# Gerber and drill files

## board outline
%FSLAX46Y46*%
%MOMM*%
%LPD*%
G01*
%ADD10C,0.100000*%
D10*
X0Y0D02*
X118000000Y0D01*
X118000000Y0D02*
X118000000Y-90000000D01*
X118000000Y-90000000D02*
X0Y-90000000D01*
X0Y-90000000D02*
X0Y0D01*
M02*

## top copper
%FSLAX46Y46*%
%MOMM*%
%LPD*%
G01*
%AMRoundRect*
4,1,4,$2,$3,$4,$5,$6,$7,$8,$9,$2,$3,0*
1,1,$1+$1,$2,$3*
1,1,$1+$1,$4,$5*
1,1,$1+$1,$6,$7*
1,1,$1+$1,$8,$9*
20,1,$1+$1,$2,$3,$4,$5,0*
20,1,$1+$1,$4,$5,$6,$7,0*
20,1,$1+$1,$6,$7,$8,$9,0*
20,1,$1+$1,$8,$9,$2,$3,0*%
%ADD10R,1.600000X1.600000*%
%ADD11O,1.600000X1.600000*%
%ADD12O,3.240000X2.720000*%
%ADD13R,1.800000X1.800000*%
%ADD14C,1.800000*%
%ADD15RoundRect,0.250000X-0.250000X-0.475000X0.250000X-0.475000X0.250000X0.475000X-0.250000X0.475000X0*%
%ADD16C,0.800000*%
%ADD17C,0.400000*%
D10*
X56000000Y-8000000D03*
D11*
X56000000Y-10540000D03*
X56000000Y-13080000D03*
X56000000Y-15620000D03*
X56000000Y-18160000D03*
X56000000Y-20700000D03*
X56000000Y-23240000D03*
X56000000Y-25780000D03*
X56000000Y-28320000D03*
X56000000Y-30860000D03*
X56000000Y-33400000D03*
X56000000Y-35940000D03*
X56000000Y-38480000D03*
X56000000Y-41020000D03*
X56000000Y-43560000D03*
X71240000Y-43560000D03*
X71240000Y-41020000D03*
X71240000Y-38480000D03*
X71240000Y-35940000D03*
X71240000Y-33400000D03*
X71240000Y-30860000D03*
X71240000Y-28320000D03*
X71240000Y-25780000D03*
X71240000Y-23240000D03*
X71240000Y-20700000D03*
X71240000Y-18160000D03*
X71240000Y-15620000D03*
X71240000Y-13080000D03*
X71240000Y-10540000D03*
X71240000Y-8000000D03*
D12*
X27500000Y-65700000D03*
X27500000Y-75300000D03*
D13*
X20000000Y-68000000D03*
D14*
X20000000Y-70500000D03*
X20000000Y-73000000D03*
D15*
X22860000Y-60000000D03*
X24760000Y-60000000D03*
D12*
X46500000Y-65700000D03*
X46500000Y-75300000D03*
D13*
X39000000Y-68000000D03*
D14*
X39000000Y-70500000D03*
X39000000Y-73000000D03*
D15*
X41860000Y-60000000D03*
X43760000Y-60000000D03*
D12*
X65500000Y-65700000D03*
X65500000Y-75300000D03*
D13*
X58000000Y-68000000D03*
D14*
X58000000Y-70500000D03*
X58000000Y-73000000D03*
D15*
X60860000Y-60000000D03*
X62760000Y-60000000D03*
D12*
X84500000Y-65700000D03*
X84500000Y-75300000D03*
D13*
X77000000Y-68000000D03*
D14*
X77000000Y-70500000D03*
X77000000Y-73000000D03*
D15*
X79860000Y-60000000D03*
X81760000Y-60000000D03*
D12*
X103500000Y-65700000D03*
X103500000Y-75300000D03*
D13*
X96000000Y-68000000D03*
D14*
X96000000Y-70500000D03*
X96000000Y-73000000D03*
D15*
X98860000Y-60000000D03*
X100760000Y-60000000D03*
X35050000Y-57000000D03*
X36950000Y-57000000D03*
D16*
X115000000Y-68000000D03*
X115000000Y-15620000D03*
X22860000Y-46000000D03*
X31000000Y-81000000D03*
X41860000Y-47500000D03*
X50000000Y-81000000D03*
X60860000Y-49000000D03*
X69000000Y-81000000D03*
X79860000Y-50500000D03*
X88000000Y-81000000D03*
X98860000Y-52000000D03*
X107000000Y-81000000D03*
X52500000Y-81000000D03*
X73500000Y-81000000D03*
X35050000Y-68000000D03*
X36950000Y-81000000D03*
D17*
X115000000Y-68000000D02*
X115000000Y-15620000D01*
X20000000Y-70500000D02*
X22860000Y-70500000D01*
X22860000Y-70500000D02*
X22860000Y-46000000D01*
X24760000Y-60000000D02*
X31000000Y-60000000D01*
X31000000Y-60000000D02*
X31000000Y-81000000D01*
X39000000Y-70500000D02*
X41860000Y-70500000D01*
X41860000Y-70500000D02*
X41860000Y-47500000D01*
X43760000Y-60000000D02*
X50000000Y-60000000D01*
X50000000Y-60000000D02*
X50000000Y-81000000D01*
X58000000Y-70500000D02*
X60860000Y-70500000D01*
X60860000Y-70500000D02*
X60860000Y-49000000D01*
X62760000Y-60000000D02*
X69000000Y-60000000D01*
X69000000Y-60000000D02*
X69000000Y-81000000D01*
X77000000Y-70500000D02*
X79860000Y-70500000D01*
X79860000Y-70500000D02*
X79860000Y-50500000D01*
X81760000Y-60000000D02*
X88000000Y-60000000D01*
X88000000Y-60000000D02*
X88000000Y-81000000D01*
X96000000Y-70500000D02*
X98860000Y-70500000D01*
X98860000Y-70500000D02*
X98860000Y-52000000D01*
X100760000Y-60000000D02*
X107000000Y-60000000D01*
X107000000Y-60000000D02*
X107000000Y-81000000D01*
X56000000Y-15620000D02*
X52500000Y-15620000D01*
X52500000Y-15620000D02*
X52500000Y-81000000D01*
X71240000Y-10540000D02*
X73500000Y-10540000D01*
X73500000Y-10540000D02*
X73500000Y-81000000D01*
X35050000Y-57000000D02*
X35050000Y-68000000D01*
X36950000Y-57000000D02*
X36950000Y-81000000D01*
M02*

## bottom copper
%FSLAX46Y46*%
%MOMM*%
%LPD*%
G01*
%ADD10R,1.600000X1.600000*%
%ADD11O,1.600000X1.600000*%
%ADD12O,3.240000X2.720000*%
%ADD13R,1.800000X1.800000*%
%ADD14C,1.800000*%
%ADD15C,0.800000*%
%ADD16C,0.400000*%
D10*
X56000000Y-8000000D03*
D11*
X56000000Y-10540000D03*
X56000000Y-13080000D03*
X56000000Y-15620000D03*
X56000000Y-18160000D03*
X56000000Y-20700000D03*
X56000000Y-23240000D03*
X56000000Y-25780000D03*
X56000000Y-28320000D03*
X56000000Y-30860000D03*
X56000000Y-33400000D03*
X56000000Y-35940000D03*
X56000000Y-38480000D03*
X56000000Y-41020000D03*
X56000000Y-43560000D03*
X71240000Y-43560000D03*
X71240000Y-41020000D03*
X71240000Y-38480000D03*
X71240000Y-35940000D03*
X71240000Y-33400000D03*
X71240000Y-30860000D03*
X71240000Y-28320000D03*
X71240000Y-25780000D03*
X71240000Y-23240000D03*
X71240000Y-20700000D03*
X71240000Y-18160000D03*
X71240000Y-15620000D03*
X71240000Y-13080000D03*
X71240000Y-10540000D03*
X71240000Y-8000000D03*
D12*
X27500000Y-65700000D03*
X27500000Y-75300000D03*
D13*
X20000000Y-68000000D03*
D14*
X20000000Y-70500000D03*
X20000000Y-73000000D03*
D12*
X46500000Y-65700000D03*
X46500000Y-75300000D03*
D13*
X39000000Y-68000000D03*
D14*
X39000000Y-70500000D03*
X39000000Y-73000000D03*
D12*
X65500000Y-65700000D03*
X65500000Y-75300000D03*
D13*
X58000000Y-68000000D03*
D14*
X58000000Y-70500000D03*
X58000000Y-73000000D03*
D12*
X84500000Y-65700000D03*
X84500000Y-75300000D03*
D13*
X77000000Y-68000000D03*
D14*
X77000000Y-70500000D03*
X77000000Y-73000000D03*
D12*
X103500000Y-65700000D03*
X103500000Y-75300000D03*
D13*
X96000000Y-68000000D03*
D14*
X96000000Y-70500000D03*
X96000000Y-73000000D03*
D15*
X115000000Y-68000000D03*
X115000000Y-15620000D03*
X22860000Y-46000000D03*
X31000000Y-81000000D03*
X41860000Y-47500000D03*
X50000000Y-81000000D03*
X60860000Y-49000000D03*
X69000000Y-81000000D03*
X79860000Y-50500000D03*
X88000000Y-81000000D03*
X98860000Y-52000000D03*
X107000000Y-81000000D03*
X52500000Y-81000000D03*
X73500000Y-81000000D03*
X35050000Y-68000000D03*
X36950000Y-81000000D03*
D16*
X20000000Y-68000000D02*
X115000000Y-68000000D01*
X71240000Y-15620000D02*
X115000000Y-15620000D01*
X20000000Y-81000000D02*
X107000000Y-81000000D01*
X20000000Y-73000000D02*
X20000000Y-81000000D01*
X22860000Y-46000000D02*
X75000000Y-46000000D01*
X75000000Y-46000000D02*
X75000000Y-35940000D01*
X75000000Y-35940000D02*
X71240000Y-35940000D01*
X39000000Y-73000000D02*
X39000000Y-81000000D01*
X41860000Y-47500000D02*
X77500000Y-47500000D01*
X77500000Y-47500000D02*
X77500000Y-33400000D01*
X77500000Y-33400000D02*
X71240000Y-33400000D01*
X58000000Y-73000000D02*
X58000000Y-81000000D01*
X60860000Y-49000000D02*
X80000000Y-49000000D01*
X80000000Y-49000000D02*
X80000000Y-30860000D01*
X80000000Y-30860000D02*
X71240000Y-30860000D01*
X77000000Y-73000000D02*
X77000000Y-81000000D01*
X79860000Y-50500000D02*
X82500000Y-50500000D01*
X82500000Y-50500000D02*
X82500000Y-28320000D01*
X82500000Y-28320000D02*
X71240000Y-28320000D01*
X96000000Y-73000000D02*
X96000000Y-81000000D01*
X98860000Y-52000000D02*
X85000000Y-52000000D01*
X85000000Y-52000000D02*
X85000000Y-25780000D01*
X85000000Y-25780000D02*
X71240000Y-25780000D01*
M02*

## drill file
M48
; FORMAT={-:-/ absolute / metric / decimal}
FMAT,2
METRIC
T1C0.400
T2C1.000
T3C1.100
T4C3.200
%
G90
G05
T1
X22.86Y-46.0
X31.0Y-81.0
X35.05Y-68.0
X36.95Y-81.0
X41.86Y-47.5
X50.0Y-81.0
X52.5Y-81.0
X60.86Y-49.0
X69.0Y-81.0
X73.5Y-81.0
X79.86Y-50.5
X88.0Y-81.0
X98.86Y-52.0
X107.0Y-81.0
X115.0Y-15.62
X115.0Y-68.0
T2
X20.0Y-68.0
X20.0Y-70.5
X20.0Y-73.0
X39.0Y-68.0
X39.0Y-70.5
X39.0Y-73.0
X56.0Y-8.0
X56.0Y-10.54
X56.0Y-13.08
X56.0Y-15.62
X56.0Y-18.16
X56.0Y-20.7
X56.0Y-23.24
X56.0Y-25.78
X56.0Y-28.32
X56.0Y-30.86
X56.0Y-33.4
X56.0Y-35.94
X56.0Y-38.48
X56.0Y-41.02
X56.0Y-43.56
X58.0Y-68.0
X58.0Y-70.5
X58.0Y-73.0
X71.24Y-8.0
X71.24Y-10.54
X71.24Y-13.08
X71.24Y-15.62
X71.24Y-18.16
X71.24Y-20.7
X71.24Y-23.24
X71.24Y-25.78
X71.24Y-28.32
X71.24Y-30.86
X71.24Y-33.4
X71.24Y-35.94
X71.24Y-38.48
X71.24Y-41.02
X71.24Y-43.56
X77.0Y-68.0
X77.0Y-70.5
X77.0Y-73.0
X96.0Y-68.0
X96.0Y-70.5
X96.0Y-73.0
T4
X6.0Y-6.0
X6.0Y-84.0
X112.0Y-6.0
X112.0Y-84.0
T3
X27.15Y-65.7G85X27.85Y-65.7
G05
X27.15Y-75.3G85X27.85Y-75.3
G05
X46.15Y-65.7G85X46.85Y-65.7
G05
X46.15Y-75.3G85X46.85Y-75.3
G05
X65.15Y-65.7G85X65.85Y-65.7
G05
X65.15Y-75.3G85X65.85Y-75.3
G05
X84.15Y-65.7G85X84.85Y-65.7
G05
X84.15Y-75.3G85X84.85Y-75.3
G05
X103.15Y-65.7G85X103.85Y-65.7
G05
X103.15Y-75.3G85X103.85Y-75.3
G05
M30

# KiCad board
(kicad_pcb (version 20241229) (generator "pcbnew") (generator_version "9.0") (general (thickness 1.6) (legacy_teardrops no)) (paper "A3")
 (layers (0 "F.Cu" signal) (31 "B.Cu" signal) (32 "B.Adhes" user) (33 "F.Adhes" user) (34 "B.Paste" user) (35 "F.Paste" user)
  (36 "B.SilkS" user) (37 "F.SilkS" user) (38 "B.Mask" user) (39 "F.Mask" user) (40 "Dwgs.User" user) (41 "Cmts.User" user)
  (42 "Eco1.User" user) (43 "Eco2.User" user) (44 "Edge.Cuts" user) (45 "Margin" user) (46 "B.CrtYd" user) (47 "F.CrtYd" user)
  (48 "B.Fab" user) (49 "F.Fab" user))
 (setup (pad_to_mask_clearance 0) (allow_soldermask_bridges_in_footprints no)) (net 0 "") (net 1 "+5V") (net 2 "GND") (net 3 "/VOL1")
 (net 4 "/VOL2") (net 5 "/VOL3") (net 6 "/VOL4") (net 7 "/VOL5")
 (gr_line (start 0 0) (end 118 0) (stroke (width 0.1) (type solid)) (layer "Edge.Cuts"))
 (gr_line (start 118 0) (end 118 90) (stroke (width 0.1) (type solid)) (layer "Edge.Cuts"))
 (gr_line (start 118 90) (end 0 90) (stroke (width 0.1) (type solid)) (layer "Edge.Cuts"))
 (gr_line (start 0 90) (end 0 0) (stroke (width 0.1) (type solid)) (layer "Edge.Cuts"))
 (segment (start 20 68) (end 115 68) (width 0.4) (layer "B.Cu") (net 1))
 (segment (start 71.24 15.62) (end 115 15.62) (width 0.4) (layer "B.Cu") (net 1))
 (segment (start 20 81) (end 107 81) (width 0.4) (layer "B.Cu") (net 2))
 (segment (start 20 73) (end 20 81) (width 0.4) (layer "B.Cu") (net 2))
 (segment (start 22.86 46) (end 75 46) (width 0.4) (layer "B.Cu") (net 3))
 (segment (start 75 46) (end 75 35.94) (width 0.4) (layer "B.Cu") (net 3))
 (segment (start 75 35.94) (end 71.24 35.94) (width 0.4) (layer "B.Cu") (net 3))
 (segment (start 39 73) (end 39 81) (width 0.4) (layer "B.Cu") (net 2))
 (segment (start 41.86 47.5) (end 77.5 47.5) (width 0.4) (layer "B.Cu") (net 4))
 (segment (start 77.5 47.5) (end 77.5 33.4) (width 0.4) (layer "B.Cu") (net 4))
 (segment (start 77.5 33.4) (end 71.24 33.4) (width 0.4) (layer "B.Cu") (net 4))
 (segment (start 58 73) (end 58 81) (width 0.4) (layer "B.Cu") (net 2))
 (segment (start 60.86 49) (end 80 49) (width 0.4) (layer "B.Cu") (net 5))
 (segment (start 80 49) (end 80 30.86) (width 0.4) (layer "B.Cu") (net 5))
 (segment (start 80 30.86) (end 71.24 30.86) (width 0.4) (layer "B.Cu") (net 5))
 (segment (start 77 73) (end 77 81) (width 0.4) (layer "B.Cu") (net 2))
 (segment (start 79.86 50.5) (end 82.5 50.5) (width 0.4) (layer "B.Cu") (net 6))
 (segment (start 82.5 50.5) (end 82.5 28.32) (width 0.4) (layer "B.Cu") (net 6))
 (segment (start 82.5 28.32) (end 71.24 28.32) (width 0.4) (layer "B.Cu") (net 6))
 (segment (start 96 73) (end 96 81) (width 0.4) (layer "B.Cu") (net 2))
 (segment (start 98.86 52) (end 85 52) (width 0.4) (layer "B.Cu") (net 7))
 (segment (start 85 52) (end 85 25.78) (width 0.4) (layer "B.Cu") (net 7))
 (segment (start 85 25.78) (end 71.24 25.78) (width 0.4) (layer "B.Cu") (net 7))
 (segment (start 115 68) (end 115 15.62) (width 0.4) (layer "F.Cu") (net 1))
 (segment (start 20 70.5) (end 22.86 70.5) (width 0.4) (layer "F.Cu") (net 3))
 (segment (start 22.86 70.5) (end 22.86 46) (width 0.4) (layer "F.Cu") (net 3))
 (segment (start 24.76 60) (end 31 60) (width 0.4) (layer "F.Cu") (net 2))
 (segment (start 31 60) (end 31 81) (width 0.4) (layer "F.Cu") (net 2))
 (segment (start 39 70.5) (end 41.86 70.5) (width 0.4) (layer "F.Cu") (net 4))
 (segment (start 41.86 70.5) (end 41.86 47.5) (width 0.4) (layer "F.Cu") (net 4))
 (segment (start 43.76 60) (end 50 60) (width 0.4) (layer "F.Cu") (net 2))
 (segment (start 50 60) (end 50 81) (width 0.4) (layer "F.Cu") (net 2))
 (segment (start 58 70.5) (end 60.86 70.5) (width 0.4) (layer "F.Cu") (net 5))
 (segment (start 60.86 70.5) (end 60.86 49) (width 0.4) (layer "F.Cu") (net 5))
 (segment (start 62.76 60) (end 69 60) (width 0.4) (layer "F.Cu") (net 2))
 (segment (start 69 60) (end 69 81) (width 0.4) (layer "F.Cu") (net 2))
 (segment (start 77 70.5) (end 79.86 70.5) (width 0.4) (layer "F.Cu") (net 6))
 (segment (start 79.86 70.5) (end 79.86 50.5) (width 0.4) (layer "F.Cu") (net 6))
 (segment (start 81.76 60) (end 88 60) (width 0.4) (layer "F.Cu") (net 2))
 (segment (start 88 60) (end 88 81) (width 0.4) (layer "F.Cu") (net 2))
 (segment (start 96 70.5) (end 98.86 70.5) (width 0.4) (layer "F.Cu") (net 7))
 (segment (start 98.86 70.5) (end 98.86 52) (width 0.4) (layer "F.Cu") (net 7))
 (segment (start 100.76 60) (end 107 60) (width 0.4) (layer "F.Cu") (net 2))
 (segment (start 107 60) (end 107 81) (width 0.4) (layer "F.Cu") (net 2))
 (segment (start 56 15.62) (end 52.5 15.62) (width 0.4) (layer "F.Cu") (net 2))
 (segment (start 52.5 15.62) (end 52.5 81) (width 0.4) (layer "F.Cu") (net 2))
 (segment (start 71.24 10.54) (end 73.5 10.54) (width 0.4) (layer "F.Cu") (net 2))
 (segment (start 73.5 10.54) (end 73.5 81) (width 0.4) (layer "F.Cu") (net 2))
 (segment (start 35.05 57) (end 35.05 68) (width 0.4) (layer "F.Cu") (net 1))
 (segment (start 36.95 57) (end 36.95 81) (width 0.4) (layer "F.Cu") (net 2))
 (via (at 115 68) (size 0.8) (drill 0.4) (layers "F.Cu" "B.Cu") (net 1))
 (via (at 115 15.62) (size 0.8) (drill 0.4) (layers "F.Cu" "B.Cu") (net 1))
 (via (at 22.86 46) (size 0.8) (drill 0.4) (layers "F.Cu" "B.Cu") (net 3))
 (via (at 31 81) (size 0.8) (drill 0.4) (layers "F.Cu" "B.Cu") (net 2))
 (via (at 41.86 47.5) (size 0.8) (drill 0.4) (layers "F.Cu" "B.Cu") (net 4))
 (via (at 50 81) (size 0.8) (drill 0.4) (layers "F.Cu" "B.Cu") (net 2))
 (via (at 60.86 49) (size 0.8) (drill 0.4) (layers "F.Cu" "B.Cu") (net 5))
 (via (at 69 81) (size 0.8) (drill 0.4) (layers "F.Cu" "B.Cu") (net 2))
 (via (at 79.86 50.5) (size 0.8) (drill 0.4) (layers "F.Cu" "B.Cu") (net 6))
 (via (at 88 81) (size 0.8) (drill 0.4) (layers "F.Cu" "B.Cu") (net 2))
 (via (at 98.86 52) (size 0.8) (drill 0.4) (layers "F.Cu" "B.Cu") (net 7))
 (via (at 107 81) (size 0.8) (drill 0.4) (layers "F.Cu" "B.Cu") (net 2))
 (via (at 52.5 81) (size 0.8) (drill 0.4) (layers "F.Cu" "B.Cu") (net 2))
 (via (at 73.5 81) (size 0.8) (drill 0.4) (layers "F.Cu" "B.Cu") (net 2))
 (via (at 35.05 68) (size 0.8) (drill 0.4) (layers "F.Cu" "B.Cu") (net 1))
 (via (at 36.95 81) (size 0.8) (drill 0.4) (layers "F.Cu" "B.Cu") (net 2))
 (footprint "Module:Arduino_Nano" (at 56 8 0) (layer "F.Cu")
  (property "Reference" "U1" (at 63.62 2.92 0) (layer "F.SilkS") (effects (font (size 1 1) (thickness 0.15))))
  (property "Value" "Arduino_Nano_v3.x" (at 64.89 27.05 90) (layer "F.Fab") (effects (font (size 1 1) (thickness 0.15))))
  (pad "1" thru_hole rect (at 0 0) (size 1.6 1.6) (drill 1) (layers "*.Cu" "*.Mask") (remove_unused_layers no))
  (pad "2" thru_hole oval (at 0 2.54) (size 1.6 1.6) (drill 1) (layers "*.Cu" "*.Mask") (remove_unused_layers no))
  (pad "3" thru_hole oval (at 0 5.08) (size 1.6 1.6) (drill 1) (layers "*.Cu" "*.Mask") (remove_unused_layers no))
  (pad "4" thru_hole oval (at 0 7.62) (size 1.6 1.6) (drill 1) (layers "*.Cu" "*.Mask") (remove_unused_layers no) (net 2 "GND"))
  (pad "5" thru_hole oval (at 0 10.16) (size 1.6 1.6) (drill 1) (layers "*.Cu" "*.Mask") (remove_unused_layers no))
  (pad "6" thru_hole oval (at 0 12.7) (size 1.6 1.6) (drill 1) (layers "*.Cu" "*.Mask") (remove_unused_layers no))
  (pad "7" thru_hole oval (at 0 15.24) (size 1.6 1.6) (drill 1) (layers "*.Cu" "*.Mask") (remove_unused_layers no))
  (pad "8" thru_hole oval (at 0 17.78) (size 1.6 1.6) (drill 1) (layers "*.Cu" "*.Mask") (remove_unused_layers no))
  (pad "9" thru_hole oval (at 0 20.32) (size 1.6 1.6) (drill 1) (layers "*.Cu" "*.Mask") (remove_unused_layers no))
  (pad "10" thru_hole oval (at 0 22.86) (size 1.6 1.6) (drill 1) (layers "*.Cu" "*.Mask") (remove_unused_layers no))
  (pad "11" thru_hole oval (at 0 25.4) (size 1.6 1.6) (drill 1) (layers "*.Cu" "*.Mask") (remove_unused_layers no))
  (pad "12" thru_hole oval (at 0 27.94) (size 1.6 1.6) (drill 1) (layers "*.Cu" "*.Mask") (remove_unused_layers no))
  (pad "13" thru_hole oval (at 0 30.48) (size 1.6 1.6) (drill 1) (layers "*.Cu" "*.Mask") (remove_unused_layers no))
  (pad "14" thru_hole oval (at 0 33.02) (size 1.6 1.6) (drill 1) (layers "*.Cu" "*.Mask") (remove_unused_layers no))
  (pad "15" thru_hole oval (at 0 35.56) (size 1.6 1.6) (drill 1) (layers "*.Cu" "*.Mask") (remove_unused_layers no))
  (pad "16" thru_hole oval (at 15.24 35.56) (size 1.6 1.6) (drill 1) (layers "*.Cu" "*.Mask") (remove_unused_layers no))
  (pad "17" thru_hole oval (at 15.24 33.02) (size 1.6 1.6) (drill 1) (layers "*.Cu" "*.Mask") (remove_unused_layers no))
  (pad "18" thru_hole oval (at 15.24 30.48) (size 1.6 1.6) (drill 1) (layers "*.Cu" "*.Mask") (remove_unused_layers no))
  (pad "19" thru_hole oval (at 15.24 27.94) (size 1.6 1.6) (drill 1) (layers "*.Cu" "*.Mask") (remove_unused_layers no) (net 3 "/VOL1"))
  (pad "20" thru_hole oval (at 15.24 25.4) (size 1.6 1.6) (drill 1) (layers "*.Cu" "*.Mask") (remove_unused_layers no) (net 4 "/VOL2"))
  (pad "21" thru_hole oval (at 15.24 22.86) (size 1.6 1.6) (drill 1) (layers "*.Cu" "*.Mask") (remove_unused_layers no) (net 5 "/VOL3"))
  (pad "22" thru_hole oval (at 15.24 20.32) (size 1.6 1.6) (drill 1) (layers "*.Cu" "*.Mask") (remove_unused_layers no) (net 6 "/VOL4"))
  (pad "23" thru_hole oval (at 15.24 17.78) (size 1.6 1.6) (drill 1) (layers "*.Cu" "*.Mask") (remove_unused_layers no) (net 7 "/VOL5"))
  (pad "24" thru_hole oval (at 15.24 15.24) (size 1.6 1.6) (drill 1) (layers "*.Cu" "*.Mask") (remove_unused_layers no))
  (pad "25" thru_hole oval (at 15.24 12.7) (size 1.6 1.6) (drill 1) (layers "*.Cu" "*.Mask") (remove_unused_layers no))
  (pad "26" thru_hole oval (at 15.24 10.16) (size 1.6 1.6) (drill 1) (layers "*.Cu" "*.Mask") (remove_unused_layers no))
  (pad "27" thru_hole oval (at 15.24 7.62) (size 1.6 1.6) (drill 1) (layers "*.Cu" "*.Mask") (remove_unused_layers no) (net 1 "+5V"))
  (pad "28" thru_hole oval (at 15.24 5.08) (size 1.6 1.6) (drill 1) (layers "*.Cu" "*.Mask") (remove_unused_layers no))
  (pad "29" thru_hole oval (at 15.24 2.54) (size 1.6 1.6) (drill 1) (layers "*.Cu" "*.Mask") (remove_unused_layers no) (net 2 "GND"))
  (pad "30" thru_hole oval (at 15.24 0) (size 1.6 1.6) (drill 1) (layers "*.Cu" "*.Mask") (remove_unused_layers no)))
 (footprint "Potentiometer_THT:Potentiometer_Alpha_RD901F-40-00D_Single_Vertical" (at 20 68 0) (layer "F.Cu")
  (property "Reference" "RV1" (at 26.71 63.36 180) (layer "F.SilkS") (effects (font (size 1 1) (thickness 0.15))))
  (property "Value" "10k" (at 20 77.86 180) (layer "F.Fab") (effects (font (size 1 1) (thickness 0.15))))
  (pad "" thru_hole oval (at 7.5 -2.3 90) (size 2.72 3.24) (drill oval 1.1 1.8) (layers "*.Cu" "*.Mask") (remove_unused_layers no))
  (pad "" thru_hole oval (at 7.5 7.3 90) (size 2.72 3.24) (drill oval 1.1 1.8) (layers "*.Cu" "*.Mask") (remove_unused_layers no))
  (pad "1" thru_hole rect (at 0 0 90) (size 1.8 1.8) (drill 1) (layers "*.Cu" "*.Mask") (remove_unused_layers no) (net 1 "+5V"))
  (pad "2" thru_hole circle (at 0 2.5 90) (size 1.8 1.8) (drill 1) (layers "*.Cu" "*.Mask") (remove_unused_layers no) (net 3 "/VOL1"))
  (pad "3" thru_hole circle (at 0 5 90) (size 1.8 1.8) (drill 1) (layers "*.Cu" "*.Mask") (remove_unused_layers no) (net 2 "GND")))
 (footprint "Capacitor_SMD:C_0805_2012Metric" (at 23.81 60 0) (layer "F.Cu")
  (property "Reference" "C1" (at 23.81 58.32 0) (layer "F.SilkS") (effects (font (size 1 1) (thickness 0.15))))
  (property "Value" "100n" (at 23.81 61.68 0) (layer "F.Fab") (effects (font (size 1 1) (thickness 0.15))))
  (pad "1" smd roundrect (at -0.95 0) (size 1 1.45) (layers "F.Cu" "F.Mask" "F.Paste") (roundrect_rratio 0.25) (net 3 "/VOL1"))
  (pad "2" smd roundrect (at 0.95 0) (size 1 1.45) (layers "F.Cu" "F.Mask" "F.Paste") (roundrect_rratio 0.25) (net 2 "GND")))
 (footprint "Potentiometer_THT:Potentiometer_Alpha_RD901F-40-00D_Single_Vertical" (at 39 68 0) (layer "F.Cu")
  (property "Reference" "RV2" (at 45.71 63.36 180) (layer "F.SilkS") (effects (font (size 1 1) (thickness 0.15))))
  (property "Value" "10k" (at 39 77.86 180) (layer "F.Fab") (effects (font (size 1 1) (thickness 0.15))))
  (pad "" thru_hole oval (at 7.5 -2.3 90) (size 2.72 3.24) (drill oval 1.1 1.8) (layers "*.Cu" "*.Mask") (remove_unused_layers no))
  (pad "" thru_hole oval (at 7.5 7.3 90) (size 2.72 3.24) (drill oval 1.1 1.8) (layers "*.Cu" "*.Mask") (remove_unused_layers no))
  (pad "1" thru_hole rect (at 0 0 90) (size 1.8 1.8) (drill 1) (layers "*.Cu" "*.Mask") (remove_unused_layers no) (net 1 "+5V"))
  (pad "2" thru_hole circle (at 0 2.5 90) (size 1.8 1.8) (drill 1) (layers "*.Cu" "*.Mask") (remove_unused_layers no) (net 4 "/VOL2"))
  (pad "3" thru_hole circle (at 0 5 90) (size 1.8 1.8) (drill 1) (layers "*.Cu" "*.Mask") (remove_unused_layers no) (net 2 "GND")))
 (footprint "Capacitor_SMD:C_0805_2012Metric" (at 42.81 60 0) (layer "F.Cu")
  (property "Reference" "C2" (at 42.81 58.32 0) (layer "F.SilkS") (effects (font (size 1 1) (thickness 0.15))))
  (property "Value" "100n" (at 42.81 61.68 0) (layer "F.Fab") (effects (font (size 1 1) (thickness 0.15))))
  (pad "1" smd roundrect (at -0.95 0) (size 1 1.45) (layers "F.Cu" "F.Mask" "F.Paste") (roundrect_rratio 0.25) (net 4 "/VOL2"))
  (pad "2" smd roundrect (at 0.95 0) (size 1 1.45) (layers "F.Cu" "F.Mask" "F.Paste") (roundrect_rratio 0.25) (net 2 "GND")))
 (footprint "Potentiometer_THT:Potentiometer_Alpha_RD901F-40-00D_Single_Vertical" (at 58 68 0) (layer "F.Cu")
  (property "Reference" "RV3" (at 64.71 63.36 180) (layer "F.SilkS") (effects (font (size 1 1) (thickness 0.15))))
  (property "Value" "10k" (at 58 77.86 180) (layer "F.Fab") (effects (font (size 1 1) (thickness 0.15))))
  (pad "" thru_hole oval (at 7.5 -2.3 90) (size 2.72 3.24) (drill oval 1.1 1.8) (layers "*.Cu" "*.Mask") (remove_unused_layers no))
  (pad "" thru_hole oval (at 7.5 7.3 90) (size 2.72 3.24) (drill oval 1.1 1.8) (layers "*.Cu" "*.Mask") (remove_unused_layers no))
  (pad "1" thru_hole rect (at 0 0 90) (size 1.8 1.8) (drill 1) (layers "*.Cu" "*.Mask") (remove_unused_layers no) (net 1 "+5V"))
  (pad "2" thru_hole circle (at 0 2.5 90) (size 1.8 1.8) (drill 1) (layers "*.Cu" "*.Mask") (remove_unused_layers no) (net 5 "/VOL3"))
  (pad "3" thru_hole circle (at 0 5 90) (size 1.8 1.8) (drill 1) (layers "*.Cu" "*.Mask") (remove_unused_layers no) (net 2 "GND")))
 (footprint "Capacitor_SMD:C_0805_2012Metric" (at 61.81 60 0) (layer "F.Cu")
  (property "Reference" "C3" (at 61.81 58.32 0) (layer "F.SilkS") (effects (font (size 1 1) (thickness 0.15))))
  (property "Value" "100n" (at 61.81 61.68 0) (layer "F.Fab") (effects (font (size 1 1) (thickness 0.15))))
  (pad "1" smd roundrect (at -0.95 0) (size 1 1.45) (layers "F.Cu" "F.Mask" "F.Paste") (roundrect_rratio 0.25) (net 5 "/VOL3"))
  (pad "2" smd roundrect (at 0.95 0) (size 1 1.45) (layers "F.Cu" "F.Mask" "F.Paste") (roundrect_rratio 0.25) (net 2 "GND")))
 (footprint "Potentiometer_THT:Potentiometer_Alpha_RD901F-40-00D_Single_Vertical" (at 77 68 0) (layer "F.Cu")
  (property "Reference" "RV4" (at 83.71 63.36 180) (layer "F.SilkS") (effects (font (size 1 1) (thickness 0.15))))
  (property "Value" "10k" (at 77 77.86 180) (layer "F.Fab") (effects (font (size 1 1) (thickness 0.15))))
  (pad "" thru_hole oval (at 7.5 -2.3 90) (size 2.72 3.24) (drill oval 1.1 1.8) (layers "*.Cu" "*.Mask") (remove_unused_layers no))
  (pad "" thru_hole oval (at 7.5 7.3 90) (size 2.72 3.24) (drill oval 1.1 1.8) (layers "*.Cu" "*.Mask") (remove_unused_layers no))
  (pad "1" thru_hole rect (at 0 0 90) (size 1.8 1.8) (drill 1) (layers "*.Cu" "*.Mask") (remove_unused_layers no) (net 1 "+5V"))
  (pad "2" thru_hole circle (at 0 2.5 90) (size 1.8 1.8) (drill 1) (layers "*.Cu" "*.Mask") (remove_unused_layers no) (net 6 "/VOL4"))
  (pad "3" thru_hole circle (at 0 5 90) (size 1.8 1.8) (drill 1) (layers "*.Cu" "*.Mask") (remove_unused_layers no) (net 2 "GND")))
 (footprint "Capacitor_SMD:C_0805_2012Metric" (at 80.81 60 0) (layer "F.Cu")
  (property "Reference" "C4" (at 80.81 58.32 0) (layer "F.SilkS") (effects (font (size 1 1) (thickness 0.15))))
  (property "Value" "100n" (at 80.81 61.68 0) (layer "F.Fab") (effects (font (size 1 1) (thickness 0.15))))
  (pad "1" smd roundrect (at -0.95 0) (size 1 1.45) (layers "F.Cu" "F.Mask" "F.Paste") (roundrect_rratio 0.25) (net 6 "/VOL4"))
  (pad "2" smd roundrect (at 0.95 0) (size 1 1.45) (layers "F.Cu" "F.Mask" "F.Paste") (roundrect_rratio 0.25) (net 2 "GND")))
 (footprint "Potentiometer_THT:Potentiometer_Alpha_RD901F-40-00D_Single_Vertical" (at 96 68 0) (layer "F.Cu")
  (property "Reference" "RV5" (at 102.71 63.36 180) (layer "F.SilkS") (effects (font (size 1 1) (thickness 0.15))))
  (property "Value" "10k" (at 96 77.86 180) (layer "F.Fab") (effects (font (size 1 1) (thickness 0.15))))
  (pad "" thru_hole oval (at 7.5 -2.3 90) (size 2.72 3.24) (drill oval 1.1 1.8) (layers "*.Cu" "*.Mask") (remove_unused_layers no))
  (pad "" thru_hole oval (at 7.5 7.3 90) (size 2.72 3.24) (drill oval 1.1 1.8) (layers "*.Cu" "*.Mask") (remove_unused_layers no))
  (pad "1" thru_hole rect (at 0 0 90) (size 1.8 1.8) (drill 1) (layers "*.Cu" "*.Mask") (remove_unused_layers no) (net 1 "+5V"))
  (pad "2" thru_hole circle (at 0 2.5 90) (size 1.8 1.8) (drill 1) (layers "*.Cu" "*.Mask") (remove_unused_layers no) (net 7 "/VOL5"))
  (pad "3" thru_hole circle (at 0 5 90) (size 1.8 1.8) (drill 1) (layers "*.Cu" "*.Mask") (remove_unused_layers no) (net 2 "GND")))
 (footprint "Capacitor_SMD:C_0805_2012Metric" (at 99.81 60 0) (layer "F.Cu")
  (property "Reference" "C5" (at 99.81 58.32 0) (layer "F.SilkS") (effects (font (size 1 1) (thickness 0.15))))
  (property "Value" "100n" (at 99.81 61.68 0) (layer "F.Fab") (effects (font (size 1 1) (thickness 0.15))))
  (pad "1" smd roundrect (at -0.95 0) (size 1 1.45) (layers "F.Cu" "F.Mask" "F.Paste") (roundrect_rratio 0.25) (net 7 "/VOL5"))
  (pad "2" smd roundrect (at 0.95 0) (size 1 1.45) (layers "F.Cu" "F.Mask" "F.Paste") (roundrect_rratio 0.25) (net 2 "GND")))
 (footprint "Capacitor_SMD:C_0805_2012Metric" (at 36 57 0) (layer "F.Cu")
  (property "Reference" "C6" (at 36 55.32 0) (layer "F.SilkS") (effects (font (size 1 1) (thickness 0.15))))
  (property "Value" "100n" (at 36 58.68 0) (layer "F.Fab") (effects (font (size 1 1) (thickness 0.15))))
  (pad "1" smd roundrect (at -0.95 0) (size 1 1.45) (layers "F.Cu" "F.Mask" "F.Paste") (roundrect_rratio 0.25) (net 1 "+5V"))
  (pad "2" smd roundrect (at 0.95 0) (size 1 1.45) (layers "F.Cu" "F.Mask" "F.Paste") (roundrect_rratio 0.25) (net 2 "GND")))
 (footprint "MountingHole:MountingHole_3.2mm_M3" (at 6 6 0) (layer "F.Cu")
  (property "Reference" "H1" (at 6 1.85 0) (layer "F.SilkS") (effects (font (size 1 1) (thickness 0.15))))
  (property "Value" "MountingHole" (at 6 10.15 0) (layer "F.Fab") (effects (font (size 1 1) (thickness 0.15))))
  (pad "" np_thru_hole circle (at 0 0) (size 3.2 3.2) (drill 3.2) (layers "*.Cu" "*.Mask")))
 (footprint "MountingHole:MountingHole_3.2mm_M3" (at 112 6 0) (layer "F.Cu")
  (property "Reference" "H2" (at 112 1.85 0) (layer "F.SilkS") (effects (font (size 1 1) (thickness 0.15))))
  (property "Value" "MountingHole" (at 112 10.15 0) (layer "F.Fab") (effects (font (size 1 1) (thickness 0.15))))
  (pad "" np_thru_hole circle (at 0 0) (size 3.2 3.2) (drill 3.2) (layers "*.Cu" "*.Mask")))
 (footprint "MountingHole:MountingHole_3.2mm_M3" (at 6 84 0) (layer "F.Cu")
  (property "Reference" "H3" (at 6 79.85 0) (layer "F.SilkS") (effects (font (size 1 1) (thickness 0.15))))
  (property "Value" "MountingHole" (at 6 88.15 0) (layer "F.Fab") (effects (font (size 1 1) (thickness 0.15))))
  (pad "" np_thru_hole circle (at 0 0) (size 3.2 3.2) (drill 3.2) (layers "*.Cu" "*.Mask")))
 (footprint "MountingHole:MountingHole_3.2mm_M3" (at 112 84 0) (layer "F.Cu")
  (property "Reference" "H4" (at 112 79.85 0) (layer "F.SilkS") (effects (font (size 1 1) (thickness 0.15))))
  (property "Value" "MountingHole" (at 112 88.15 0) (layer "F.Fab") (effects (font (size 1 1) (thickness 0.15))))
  (pad "" np_thru_hole circle (at 0 0) (size 3.2 3.2) (drill 3.2) (layers "*.Cu" "*.Mask"))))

